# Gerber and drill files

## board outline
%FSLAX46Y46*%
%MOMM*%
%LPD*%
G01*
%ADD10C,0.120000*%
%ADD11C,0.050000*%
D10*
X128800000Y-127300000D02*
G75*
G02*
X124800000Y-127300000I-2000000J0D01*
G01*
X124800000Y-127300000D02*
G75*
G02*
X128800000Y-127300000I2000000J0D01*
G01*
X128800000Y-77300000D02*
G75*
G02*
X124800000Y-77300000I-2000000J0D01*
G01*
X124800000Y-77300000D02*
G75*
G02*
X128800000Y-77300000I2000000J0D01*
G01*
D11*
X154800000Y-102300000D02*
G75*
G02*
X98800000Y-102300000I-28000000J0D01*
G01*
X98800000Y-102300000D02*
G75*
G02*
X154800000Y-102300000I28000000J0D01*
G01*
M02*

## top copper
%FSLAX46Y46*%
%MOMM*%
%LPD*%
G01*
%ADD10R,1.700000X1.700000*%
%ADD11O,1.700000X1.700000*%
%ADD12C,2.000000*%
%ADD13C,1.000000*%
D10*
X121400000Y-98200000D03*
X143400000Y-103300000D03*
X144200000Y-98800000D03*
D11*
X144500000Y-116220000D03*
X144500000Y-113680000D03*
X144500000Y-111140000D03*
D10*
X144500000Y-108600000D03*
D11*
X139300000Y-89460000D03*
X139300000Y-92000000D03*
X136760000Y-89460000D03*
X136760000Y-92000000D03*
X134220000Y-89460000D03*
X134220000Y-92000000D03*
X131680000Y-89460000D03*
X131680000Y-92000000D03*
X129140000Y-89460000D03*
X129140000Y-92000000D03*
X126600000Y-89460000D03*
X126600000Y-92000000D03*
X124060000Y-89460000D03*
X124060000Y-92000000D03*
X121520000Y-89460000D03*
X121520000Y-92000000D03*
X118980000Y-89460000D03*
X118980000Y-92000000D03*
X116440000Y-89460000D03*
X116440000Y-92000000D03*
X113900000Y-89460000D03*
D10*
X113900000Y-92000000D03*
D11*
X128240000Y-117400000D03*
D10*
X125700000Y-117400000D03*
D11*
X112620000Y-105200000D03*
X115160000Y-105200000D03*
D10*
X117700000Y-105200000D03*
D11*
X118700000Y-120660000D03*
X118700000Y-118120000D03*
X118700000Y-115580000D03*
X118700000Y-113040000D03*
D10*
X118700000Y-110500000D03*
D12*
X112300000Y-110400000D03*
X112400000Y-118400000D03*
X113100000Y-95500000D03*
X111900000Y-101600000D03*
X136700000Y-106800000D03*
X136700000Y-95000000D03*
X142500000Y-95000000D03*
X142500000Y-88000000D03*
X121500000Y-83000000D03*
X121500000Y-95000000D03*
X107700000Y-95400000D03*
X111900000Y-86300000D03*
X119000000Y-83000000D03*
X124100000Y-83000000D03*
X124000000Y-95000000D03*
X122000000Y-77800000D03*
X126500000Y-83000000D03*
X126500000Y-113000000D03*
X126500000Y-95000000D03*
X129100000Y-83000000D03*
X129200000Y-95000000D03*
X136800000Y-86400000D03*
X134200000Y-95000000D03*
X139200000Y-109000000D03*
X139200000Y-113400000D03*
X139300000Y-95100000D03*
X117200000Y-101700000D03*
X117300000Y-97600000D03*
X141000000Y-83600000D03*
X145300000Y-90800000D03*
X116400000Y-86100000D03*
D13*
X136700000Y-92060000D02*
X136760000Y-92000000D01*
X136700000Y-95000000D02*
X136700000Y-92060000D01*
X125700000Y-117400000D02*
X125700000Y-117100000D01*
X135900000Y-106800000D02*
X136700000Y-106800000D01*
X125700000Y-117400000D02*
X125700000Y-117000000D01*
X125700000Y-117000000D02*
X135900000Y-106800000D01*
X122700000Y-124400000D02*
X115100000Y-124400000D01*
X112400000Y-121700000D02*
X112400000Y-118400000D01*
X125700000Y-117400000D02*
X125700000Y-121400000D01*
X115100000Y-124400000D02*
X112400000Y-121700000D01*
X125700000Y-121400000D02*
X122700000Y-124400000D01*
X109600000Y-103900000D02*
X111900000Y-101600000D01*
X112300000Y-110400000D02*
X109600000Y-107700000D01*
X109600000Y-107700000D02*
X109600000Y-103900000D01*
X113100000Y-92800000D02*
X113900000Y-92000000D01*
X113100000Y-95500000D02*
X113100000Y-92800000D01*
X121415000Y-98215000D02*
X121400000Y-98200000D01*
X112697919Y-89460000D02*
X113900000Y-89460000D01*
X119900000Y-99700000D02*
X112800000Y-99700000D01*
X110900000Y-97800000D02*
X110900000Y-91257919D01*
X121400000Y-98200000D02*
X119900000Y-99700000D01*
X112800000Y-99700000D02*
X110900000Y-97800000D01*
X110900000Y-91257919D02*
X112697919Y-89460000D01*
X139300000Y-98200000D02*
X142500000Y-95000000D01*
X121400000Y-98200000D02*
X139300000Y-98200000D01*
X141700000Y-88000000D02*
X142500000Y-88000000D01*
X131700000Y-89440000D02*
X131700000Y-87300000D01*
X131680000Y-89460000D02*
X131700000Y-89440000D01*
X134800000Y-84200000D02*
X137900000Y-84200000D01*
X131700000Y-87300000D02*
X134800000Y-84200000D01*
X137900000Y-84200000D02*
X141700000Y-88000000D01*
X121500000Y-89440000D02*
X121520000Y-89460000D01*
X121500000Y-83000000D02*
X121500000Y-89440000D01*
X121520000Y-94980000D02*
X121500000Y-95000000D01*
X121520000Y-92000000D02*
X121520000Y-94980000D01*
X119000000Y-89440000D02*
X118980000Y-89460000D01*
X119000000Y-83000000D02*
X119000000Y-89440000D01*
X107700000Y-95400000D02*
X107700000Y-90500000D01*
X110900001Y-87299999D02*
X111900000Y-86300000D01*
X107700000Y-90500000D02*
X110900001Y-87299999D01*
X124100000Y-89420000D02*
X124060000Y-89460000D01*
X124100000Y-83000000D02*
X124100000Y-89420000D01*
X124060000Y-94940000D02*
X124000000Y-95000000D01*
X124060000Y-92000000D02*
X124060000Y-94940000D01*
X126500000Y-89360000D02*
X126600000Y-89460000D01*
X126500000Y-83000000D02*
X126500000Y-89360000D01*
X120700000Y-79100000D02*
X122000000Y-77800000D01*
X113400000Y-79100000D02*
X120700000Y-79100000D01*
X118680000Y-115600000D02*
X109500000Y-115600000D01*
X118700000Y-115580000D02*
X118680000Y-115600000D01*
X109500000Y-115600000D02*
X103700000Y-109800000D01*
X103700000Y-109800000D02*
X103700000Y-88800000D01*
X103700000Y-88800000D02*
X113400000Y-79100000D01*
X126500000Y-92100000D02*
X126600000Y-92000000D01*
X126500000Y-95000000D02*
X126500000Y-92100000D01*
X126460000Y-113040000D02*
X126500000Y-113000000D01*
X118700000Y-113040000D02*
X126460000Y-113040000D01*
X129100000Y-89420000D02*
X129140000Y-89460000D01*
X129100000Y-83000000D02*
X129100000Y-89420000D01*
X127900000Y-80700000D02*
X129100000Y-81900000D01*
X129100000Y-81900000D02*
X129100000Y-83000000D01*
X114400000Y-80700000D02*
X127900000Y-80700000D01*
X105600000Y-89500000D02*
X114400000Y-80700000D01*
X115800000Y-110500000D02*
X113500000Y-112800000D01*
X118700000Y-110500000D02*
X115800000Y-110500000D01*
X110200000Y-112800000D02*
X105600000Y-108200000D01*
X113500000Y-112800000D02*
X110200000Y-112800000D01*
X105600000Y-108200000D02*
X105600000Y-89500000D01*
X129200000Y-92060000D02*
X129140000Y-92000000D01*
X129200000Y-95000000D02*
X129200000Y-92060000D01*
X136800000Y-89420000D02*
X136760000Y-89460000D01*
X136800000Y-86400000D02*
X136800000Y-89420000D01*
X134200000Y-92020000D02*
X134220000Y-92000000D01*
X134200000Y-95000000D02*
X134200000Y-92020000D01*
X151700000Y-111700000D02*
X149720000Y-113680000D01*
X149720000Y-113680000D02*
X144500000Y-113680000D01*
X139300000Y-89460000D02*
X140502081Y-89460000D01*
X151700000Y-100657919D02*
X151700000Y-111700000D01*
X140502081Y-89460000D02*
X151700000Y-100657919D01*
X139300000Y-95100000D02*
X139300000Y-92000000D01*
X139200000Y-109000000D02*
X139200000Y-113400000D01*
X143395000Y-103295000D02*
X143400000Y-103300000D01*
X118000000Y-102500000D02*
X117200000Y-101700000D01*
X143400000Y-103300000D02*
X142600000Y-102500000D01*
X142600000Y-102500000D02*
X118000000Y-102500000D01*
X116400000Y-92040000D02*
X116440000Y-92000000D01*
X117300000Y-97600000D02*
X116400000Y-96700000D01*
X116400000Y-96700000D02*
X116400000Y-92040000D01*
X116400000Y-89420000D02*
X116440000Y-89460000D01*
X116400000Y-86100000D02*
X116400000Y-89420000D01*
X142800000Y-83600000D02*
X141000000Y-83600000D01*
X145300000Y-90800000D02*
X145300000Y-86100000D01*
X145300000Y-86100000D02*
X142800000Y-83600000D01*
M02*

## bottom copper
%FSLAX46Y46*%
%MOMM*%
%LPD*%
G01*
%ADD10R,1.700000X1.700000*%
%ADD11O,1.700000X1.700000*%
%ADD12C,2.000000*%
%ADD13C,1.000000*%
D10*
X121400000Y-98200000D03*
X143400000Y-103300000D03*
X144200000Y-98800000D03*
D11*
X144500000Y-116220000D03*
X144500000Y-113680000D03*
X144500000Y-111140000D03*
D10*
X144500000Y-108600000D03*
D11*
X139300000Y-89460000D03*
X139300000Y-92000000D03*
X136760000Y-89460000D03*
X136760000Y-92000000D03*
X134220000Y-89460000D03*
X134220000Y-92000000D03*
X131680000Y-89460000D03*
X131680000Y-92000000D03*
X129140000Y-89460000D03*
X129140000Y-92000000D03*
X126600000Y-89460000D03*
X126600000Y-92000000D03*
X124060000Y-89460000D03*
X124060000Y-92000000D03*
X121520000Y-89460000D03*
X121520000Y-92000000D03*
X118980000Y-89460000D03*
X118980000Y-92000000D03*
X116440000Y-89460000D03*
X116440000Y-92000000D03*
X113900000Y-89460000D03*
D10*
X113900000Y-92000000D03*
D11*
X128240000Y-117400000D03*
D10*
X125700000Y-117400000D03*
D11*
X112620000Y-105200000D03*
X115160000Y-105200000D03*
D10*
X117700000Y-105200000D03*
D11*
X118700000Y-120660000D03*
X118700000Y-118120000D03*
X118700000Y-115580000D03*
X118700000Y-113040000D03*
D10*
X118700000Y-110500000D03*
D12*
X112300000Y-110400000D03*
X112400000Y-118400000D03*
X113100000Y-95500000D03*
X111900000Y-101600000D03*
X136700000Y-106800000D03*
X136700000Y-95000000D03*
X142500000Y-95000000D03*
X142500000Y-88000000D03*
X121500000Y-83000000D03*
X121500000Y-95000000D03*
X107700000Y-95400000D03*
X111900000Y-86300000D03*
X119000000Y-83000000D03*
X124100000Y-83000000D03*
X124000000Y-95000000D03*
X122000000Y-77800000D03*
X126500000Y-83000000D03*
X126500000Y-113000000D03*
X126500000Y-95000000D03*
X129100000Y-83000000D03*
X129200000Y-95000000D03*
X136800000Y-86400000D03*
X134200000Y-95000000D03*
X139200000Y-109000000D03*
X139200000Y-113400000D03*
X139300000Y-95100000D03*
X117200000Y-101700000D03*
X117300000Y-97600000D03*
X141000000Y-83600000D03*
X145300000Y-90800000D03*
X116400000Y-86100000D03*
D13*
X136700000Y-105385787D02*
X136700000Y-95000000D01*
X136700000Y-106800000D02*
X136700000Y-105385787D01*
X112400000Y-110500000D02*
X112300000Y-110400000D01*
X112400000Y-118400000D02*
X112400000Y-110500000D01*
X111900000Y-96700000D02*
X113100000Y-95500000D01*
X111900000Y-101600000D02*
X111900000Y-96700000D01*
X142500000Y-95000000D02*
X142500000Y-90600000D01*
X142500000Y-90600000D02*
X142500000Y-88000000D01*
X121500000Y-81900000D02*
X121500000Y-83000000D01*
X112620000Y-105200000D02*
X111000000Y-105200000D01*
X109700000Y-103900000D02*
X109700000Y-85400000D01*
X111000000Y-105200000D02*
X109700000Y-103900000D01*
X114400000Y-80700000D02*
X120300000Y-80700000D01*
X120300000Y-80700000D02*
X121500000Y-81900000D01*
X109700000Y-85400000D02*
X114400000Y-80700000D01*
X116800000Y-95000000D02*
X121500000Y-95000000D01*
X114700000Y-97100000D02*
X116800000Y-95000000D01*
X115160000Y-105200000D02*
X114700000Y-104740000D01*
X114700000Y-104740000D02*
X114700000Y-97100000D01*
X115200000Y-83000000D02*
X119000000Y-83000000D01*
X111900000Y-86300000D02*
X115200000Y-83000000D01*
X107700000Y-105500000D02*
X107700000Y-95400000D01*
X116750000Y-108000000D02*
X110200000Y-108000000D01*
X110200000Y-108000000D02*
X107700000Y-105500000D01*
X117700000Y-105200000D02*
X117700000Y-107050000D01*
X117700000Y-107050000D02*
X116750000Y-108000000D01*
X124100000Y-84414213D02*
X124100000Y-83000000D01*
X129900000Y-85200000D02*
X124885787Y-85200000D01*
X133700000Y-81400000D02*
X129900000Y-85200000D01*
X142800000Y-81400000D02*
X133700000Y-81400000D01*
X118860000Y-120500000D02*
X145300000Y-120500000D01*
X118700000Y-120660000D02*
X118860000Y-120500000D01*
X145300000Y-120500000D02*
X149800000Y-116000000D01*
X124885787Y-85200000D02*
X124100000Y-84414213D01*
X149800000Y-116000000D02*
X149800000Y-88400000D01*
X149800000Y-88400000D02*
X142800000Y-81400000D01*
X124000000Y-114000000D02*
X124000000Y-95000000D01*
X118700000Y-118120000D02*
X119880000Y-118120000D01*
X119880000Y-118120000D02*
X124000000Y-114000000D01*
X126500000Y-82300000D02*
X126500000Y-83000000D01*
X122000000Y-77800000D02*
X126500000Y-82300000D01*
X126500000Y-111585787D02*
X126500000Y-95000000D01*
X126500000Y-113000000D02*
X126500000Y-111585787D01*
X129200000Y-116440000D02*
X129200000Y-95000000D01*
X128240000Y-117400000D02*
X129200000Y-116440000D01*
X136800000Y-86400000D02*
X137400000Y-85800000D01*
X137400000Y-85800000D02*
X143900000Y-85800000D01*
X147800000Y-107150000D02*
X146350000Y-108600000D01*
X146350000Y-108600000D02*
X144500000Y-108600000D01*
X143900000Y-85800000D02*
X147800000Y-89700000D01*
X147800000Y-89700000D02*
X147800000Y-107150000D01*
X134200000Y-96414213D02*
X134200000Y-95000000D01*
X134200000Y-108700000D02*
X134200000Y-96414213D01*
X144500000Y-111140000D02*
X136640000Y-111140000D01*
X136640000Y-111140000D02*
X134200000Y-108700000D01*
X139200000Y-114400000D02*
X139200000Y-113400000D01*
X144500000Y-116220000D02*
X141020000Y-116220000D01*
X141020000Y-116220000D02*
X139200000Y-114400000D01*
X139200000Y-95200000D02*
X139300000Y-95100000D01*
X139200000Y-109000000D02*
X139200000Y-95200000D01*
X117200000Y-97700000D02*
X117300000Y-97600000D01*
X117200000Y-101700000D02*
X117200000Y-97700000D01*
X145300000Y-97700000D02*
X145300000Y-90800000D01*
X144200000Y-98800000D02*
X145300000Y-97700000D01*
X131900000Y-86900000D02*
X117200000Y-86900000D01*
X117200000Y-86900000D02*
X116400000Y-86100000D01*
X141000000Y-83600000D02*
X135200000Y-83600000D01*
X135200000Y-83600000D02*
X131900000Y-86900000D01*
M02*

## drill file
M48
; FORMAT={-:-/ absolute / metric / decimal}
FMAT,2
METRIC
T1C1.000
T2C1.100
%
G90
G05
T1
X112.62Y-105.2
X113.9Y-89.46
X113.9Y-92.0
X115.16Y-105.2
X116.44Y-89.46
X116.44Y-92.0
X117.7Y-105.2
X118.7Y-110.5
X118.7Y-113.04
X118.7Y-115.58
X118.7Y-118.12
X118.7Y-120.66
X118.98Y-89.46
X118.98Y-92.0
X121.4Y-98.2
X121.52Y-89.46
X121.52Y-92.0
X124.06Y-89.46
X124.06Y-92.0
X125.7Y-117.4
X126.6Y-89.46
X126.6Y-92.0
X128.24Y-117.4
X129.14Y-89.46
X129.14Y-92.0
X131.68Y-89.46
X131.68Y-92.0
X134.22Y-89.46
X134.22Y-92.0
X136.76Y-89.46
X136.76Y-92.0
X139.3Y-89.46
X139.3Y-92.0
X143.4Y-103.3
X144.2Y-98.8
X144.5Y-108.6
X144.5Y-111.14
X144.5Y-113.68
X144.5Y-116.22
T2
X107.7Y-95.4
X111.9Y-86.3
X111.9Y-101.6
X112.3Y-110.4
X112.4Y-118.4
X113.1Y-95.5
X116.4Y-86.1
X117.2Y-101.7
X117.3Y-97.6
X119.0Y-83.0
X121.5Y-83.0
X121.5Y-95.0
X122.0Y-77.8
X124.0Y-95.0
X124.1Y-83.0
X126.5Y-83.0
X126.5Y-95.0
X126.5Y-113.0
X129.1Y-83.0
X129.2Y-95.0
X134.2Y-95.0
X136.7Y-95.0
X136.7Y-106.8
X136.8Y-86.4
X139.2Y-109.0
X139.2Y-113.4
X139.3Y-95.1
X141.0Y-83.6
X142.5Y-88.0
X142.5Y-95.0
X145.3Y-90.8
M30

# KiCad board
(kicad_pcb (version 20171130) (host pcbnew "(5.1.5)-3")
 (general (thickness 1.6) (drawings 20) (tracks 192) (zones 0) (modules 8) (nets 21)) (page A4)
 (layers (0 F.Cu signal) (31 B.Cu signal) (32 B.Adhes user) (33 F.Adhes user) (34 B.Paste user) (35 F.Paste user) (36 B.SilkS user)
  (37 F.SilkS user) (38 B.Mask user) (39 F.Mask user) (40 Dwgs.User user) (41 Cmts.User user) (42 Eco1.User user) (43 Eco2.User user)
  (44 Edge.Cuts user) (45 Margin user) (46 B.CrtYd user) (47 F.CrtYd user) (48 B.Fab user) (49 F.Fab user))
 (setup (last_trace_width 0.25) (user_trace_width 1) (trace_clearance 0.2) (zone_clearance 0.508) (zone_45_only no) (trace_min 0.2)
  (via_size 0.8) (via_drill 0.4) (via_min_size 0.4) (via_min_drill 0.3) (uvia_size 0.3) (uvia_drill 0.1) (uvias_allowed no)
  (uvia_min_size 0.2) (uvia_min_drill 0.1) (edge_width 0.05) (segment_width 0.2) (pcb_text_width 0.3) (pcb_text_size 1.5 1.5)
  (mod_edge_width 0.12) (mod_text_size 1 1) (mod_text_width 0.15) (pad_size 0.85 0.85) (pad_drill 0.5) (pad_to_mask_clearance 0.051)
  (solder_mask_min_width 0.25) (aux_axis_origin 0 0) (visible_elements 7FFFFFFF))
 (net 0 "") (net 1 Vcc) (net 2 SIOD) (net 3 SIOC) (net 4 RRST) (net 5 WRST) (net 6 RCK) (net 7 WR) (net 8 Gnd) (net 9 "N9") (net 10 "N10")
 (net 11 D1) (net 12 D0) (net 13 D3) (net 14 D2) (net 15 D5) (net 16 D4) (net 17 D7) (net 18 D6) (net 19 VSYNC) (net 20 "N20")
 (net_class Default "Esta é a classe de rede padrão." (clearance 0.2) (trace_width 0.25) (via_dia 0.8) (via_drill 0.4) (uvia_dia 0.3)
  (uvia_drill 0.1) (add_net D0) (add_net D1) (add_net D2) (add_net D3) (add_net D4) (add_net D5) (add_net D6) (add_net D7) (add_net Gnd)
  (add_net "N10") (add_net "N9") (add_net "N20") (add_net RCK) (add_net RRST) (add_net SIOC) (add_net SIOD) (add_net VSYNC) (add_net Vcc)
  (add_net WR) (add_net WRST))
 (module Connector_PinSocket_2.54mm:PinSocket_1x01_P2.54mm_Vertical (layer F.Cu) (at 121.4 98.2)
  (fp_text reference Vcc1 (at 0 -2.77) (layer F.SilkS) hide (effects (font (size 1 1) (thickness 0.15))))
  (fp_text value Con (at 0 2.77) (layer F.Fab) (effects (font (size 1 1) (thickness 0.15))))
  (pad 1 thru_hole rect (at 0 0) (size 1.7 1.7) (drill 1) (layers *.Cu *.Mask) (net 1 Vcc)))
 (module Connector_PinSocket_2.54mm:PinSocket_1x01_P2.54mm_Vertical (layer F.Cu) (at 143.4 103.3)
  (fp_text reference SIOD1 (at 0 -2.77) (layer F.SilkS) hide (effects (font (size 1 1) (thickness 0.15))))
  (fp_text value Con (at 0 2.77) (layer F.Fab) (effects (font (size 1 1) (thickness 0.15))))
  (pad 1 thru_hole rect (at 0 0) (size 1.7 1.7) (drill 1) (layers *.Cu *.Mask) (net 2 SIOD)))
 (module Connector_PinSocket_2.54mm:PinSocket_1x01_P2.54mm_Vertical (layer F.Cu) (at 144.2 98.8)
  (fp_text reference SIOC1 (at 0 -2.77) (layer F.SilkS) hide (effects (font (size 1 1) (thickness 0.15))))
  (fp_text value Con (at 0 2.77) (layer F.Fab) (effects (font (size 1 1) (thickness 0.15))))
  (pad 1 thru_hole rect (at 0 0) (size 1.7 1.7) (drill 1) (layers *.Cu *.Mask) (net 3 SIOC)))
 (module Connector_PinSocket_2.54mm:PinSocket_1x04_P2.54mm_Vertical (layer F.Cu) (at 144.5 108.6)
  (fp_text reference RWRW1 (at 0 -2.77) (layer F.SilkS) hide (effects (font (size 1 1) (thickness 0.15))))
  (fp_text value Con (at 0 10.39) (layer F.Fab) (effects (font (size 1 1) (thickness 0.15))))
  (pad 4 thru_hole oval (at 0 7.62) (size 1.7 1.7) (drill 1) (layers *.Cu *.Mask) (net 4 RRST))
  (pad 3 thru_hole oval (at 0 5.08) (size 1.7 1.7) (drill 1) (layers *.Cu *.Mask) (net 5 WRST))
  (pad 2 thru_hole oval (at 0 2.54) (size 1.7 1.7) (drill 1) (layers *.Cu *.Mask) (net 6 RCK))
  (pad 1 thru_hole rect (at 0 0) (size 1.7 1.7) (drill 1) (layers *.Cu *.Mask) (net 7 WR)))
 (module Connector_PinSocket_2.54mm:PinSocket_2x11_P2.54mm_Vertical (layer B.Cu) (at 113.9 92 270)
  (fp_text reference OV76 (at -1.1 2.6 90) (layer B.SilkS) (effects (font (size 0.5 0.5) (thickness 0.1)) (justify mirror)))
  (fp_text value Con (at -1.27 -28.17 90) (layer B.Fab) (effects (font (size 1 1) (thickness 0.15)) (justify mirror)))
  (pad 22 thru_hole oval (at -2.54 -25.4 270) (size 1.7 1.7) (drill 1) (layers *.Cu *.Mask) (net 5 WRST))
  (pad 21 thru_hole oval (at 0 -25.4 270) (size 1.7 1.7) (drill 1) (layers *.Cu *.Mask) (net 4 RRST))
  (pad 20 thru_hole oval (at -2.54 -22.86 270) (size 1.7 1.7) (drill 1) (layers *.Cu *.Mask) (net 7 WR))
  (pad 19 thru_hole oval (at 0 -22.86 270) (size 1.7 1.7) (drill 1) (layers *.Cu *.Mask) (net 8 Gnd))
  (pad 18 thru_hole oval (at -2.54 -20.32 270) (size 1.7 1.7) (drill 1) (layers *.Cu *.Mask) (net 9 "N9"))
  (pad 17 thru_hole oval (at 0 -20.32 270) (size 1.7 1.7) (drill 1) (layers *.Cu *.Mask) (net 6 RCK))
  (pad 16 thru_hole oval (at -2.54 -17.78 270) (size 1.7 1.7) (drill 1) (layers *.Cu *.Mask) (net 1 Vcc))
  (pad 15 thru_hole oval (at 0 -17.78 270) (size 1.7 1.7) (drill 1) (layers *.Cu *.Mask) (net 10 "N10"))
  (pad 14 thru_hole oval (at -2.54 -15.24 270) (size 1.7 1.7) (drill 1) (layers *.Cu *.Mask) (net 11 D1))
  (pad 13 thru_hole oval (at 0 -15.24 270) (size 1.7 1.7) (drill 1) (layers *.Cu *.Mask) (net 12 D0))
  (pad 12 thru_hole oval (at -2.54 -12.7 270) (size 1.7 1.7) (drill 1) (layers *.Cu *.Mask) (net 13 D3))
  (pad 11 thru_hole oval (at 0 -12.7 270) (size 1.7 1.7) (drill 1) (layers *.Cu *.Mask) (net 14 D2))
  (pad 10 thru_hole oval (at -2.54 -10.16 270) (size 1.7 1.7) (drill 1) (layers *.Cu *.Mask) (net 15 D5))
  (pad 9 thru_hole oval (at 0 -10.16 270) (size 1.7 1.7) (drill 1) (layers *.Cu *.Mask) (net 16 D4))
  (pad 8 thru_hole oval (at -2.54 -7.62 270) (size 1.7 1.7) (drill 1) (layers *.Cu *.Mask) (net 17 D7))
  (pad 7 thru_hole oval (at 0 -7.62 270) (size 1.7 1.7) (drill 1) (layers *.Cu *.Mask) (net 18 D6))
  (pad 6 thru_hole oval (at -2.54 -5.08 270) (size 1.7 1.7) (drill 1) (layers *.Cu *.Mask) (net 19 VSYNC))
  (pad 5 thru_hole oval (at 0 -5.08 270) (size 1.7 1.7) (drill 1) (layers *.Cu *.Mask) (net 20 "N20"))
  (pad 4 thru_hole oval (at -2.54 -2.54 270) (size 1.7 1.7) (drill 1) (layers *.Cu *.Mask) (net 3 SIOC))
  (pad 3 thru_hole oval (at 0 -2.54 270) (size 1.7 1.7) (drill 1) (layers *.Cu *.Mask) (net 2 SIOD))
  (pad 2 thru_hole oval (at -2.54 0 270) (size 1.7 1.7) (drill 1) (layers *.Cu *.Mask) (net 1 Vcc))
  (pad 1 thru_hole rect (at 0 0 270) (size 1.7 1.7) (drill 1) (layers *.Cu *.Mask) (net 8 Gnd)))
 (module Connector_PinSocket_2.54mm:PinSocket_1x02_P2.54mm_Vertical (layer F.Cu) (at 125.7 117.4 90)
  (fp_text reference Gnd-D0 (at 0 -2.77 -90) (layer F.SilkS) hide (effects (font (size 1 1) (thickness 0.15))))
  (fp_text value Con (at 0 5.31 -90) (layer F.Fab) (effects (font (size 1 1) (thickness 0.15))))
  (pad 2 thru_hole oval (at 0 2.54 90) (size 1.7 1.7) (drill 1) (layers *.Cu *.Mask) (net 12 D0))
  (pad 1 thru_hole rect (at 0 0 90) (size 1.7 1.7) (drill 1) (layers *.Cu *.Mask) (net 8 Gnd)))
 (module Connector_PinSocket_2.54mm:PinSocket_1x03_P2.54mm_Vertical (layer F.Cu) (at 117.7 105.2 270)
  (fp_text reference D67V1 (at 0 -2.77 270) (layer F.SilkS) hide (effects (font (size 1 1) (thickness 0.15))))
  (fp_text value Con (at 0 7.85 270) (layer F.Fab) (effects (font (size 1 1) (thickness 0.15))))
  (pad 3 thru_hole oval (at 0 5.08 270) (size 1.7 1.7) (drill 1) (layers *.Cu *.Mask) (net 17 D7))
  (pad 2 thru_hole oval (at 0 2.54 270) (size 1.7 1.7) (drill 1) (layers *.Cu *.Mask) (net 18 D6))
  (pad 1 thru_hole rect (at 0 0 270) (size 1.7 1.7) (drill 1) (layers *.Cu *.Mask) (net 19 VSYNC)))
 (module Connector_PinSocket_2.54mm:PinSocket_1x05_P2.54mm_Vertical (layer F.Cu) (at 118.7 110.5)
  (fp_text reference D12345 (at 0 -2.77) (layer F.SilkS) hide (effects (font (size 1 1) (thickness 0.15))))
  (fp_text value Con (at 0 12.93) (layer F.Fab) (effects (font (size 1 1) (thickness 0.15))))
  (pad 5 thru_hole oval (at 0 10.16) (size 1.7 1.7) (drill 1) (layers *.Cu *.Mask) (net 15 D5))
  (pad 4 thru_hole oval (at 0 7.62) (size 1.7 1.7) (drill 1) (layers *.Cu *.Mask) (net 16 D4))
  (pad 3 thru_hole oval (at 0 5.08) (size 1.7 1.7) (drill 1) (layers *.Cu *.Mask) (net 13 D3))
  (pad 2 thru_hole oval (at 0 2.54) (size 1.7 1.7) (drill 1) (layers *.Cu *.Mask) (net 14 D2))
  (pad 1 thru_hole rect (at 0 0) (size 1.7 1.7) (drill 1) (layers *.Cu *.Mask) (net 11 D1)))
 (gr_circle (center 126.8 127.3) (end 128.8 127.3) (layer Edge.Cuts) (width 0.12))
 (gr_circle (center 126.8 77.3) (end 128.8 77.3) (layer Edge.Cuts) (width 0.12))
 (gr_circle (center 126.8 102.3) (end 154.8 102.3) (layer Edge.Cuts) (width 0.05))
 (via (at 112.3 110.4) (size 2) (drill 1.1) (layers F.Cu B.Cu) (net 8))
 (via (at 112.4 118.4) (size 2) (drill 1.1) (layers F.Cu B.Cu) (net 8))
 (via (at 113.1 95.5) (size 2) (drill 1.1) (layers F.Cu B.Cu) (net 8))
 (via (at 111.9 101.6) (size 2) (drill 1.1) (layers F.Cu B.Cu) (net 8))
 (via (at 136.7 106.8) (size 2) (drill 1.1) (layers F.Cu B.Cu) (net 8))
 (via (at 136.7 95) (size 2) (drill 1.1) (layers F.Cu B.Cu) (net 8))
 (segment (start 136.7 92.06) (end 136.76 92) (width 1) (layer F.Cu) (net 8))
 (segment (start 136.7 95) (end 136.7 92.06) (width 1) (layer F.Cu) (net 8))
 (segment (start 125.7 117.4) (end 125.7 117.1) (width 1) (layer F.Cu) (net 8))
 (segment (start 135.9 106.8) (end 136.7 106.8) (width 1) (layer F.Cu) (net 8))
 (segment (start 125.7 117.4) (end 125.7 117) (width 1) (layer F.Cu) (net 8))
 (segment (start 125.7 117) (end 135.9 106.8) (width 1) (layer F.Cu) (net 8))
 (segment (start 136.7 105.385787) (end 136.7 95) (width 1) (layer B.Cu) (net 8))
 (segment (start 136.7 106.8) (end 136.7 105.385787) (width 1) (layer B.Cu) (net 8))
 (segment (start 122.7 124.4) (end 115.1 124.4) (width 1) (layer F.Cu) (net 8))
 (segment (start 112.4 121.7) (end 112.4 118.4) (width 1) (layer F.Cu) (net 8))
 (segment (start 125.7 117.4) (end 125.7 121.4) (width 1) (layer F.Cu) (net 8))
 (segment (start 115.1 124.4) (end 112.4 121.7) (width 1) (layer F.Cu) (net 8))
 (segment (start 125.7 121.4) (end 122.7 124.4) (width 1) (layer F.Cu) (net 8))
 (segment (start 112.4 110.5) (end 112.3 110.4) (width 1) (layer B.Cu) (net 8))
 (segment (start 112.4 118.4) (end 112.4 110.5) (width 1) (layer B.Cu) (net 8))
 (segment (start 109.6 103.9) (end 111.9 101.6) (width 1) (layer F.Cu) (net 8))
 (segment (start 112.3 110.4) (end 109.6 107.7) (width 1) (layer F.Cu) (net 8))
 (segment (start 109.6 107.7) (end 109.6 103.9) (width 1) (layer F.Cu) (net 8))
 (segment (start 111.9 96.7) (end 113.1 95.5) (width 1) (layer B.Cu) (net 8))
 (segment (start 111.9 101.6) (end 111.9 96.7) (width 1) (layer B.Cu) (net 8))
 (segment (start 113.1 92.8) (end 113.9 92) (width 1) (layer F.Cu) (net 8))
 (segment (start 113.1 95.5) (end 113.1 92.8) (width 1) (layer F.Cu) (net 8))
 (via (at 142.5 95) (size 2) (drill 1.1) (layers F.Cu B.Cu) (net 1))
 (via (at 142.5 88) (size 2) (drill 1.1) (layers F.Cu B.Cu) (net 1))
 (segment (start 121.415 98.215) (end 121.4 98.2) (width 1) (layer F.Cu) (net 1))
 (segment (start 112.697919 89.46) (end 113.9 89.46) (width 1) (layer F.Cu) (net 1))
 (segment (start 119.9 99.7) (end 112.8 99.7) (width 1) (layer F.Cu) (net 1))
 (segment (start 110.9 97.8) (end 110.9 91.257919) (width 1) (layer F.Cu) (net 1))
 (segment (start 121.4 98.2) (end 119.9 99.7) (width 1) (layer F.Cu) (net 1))
 (segment (start 112.8 99.7) (end 110.9 97.8) (width 1) (layer F.Cu) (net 1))
 (segment (start 110.9 91.257919) (end 112.697919 89.46) (width 1) (layer F.Cu) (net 1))
 (segment (start 139.3 98.2) (end 142.5 95) (width 1) (layer F.Cu) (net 1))
 (segment (start 121.4 98.2) (end 139.3 98.2) (width 1) (layer F.Cu) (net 1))
 (segment (start 142.5 95) (end 142.5 90.6) (width 1) (layer B.Cu) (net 1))
 (segment (start 142.5 90.6) (end 142.5 88) (width 1) (layer B.Cu) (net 1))
 (segment (start 141.7 88) (end 142.5 88) (width 1) (layer F.Cu) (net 1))
 (segment (start 131.7 89.44) (end 131.7 87.3) (width 1) (layer F.Cu) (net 1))
 (segment (start 131.68 89.46) (end 131.7 89.44) (width 1) (layer F.Cu) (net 1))
 (segment (start 134.8 84.2) (end 137.9 84.2) (width 1) (layer F.Cu) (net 1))
 (segment (start 131.7 87.3) (end 134.8 84.2) (width 1) (layer F.Cu) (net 1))
 (segment (start 137.9 84.2) (end 141.7 88) (width 1) (layer F.Cu) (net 1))
 (via (at 121.5 83) (size 2) (drill 1.1) (layers F.Cu B.Cu) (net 17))
 (segment (start 121.5 89.44) (end 121.52 89.46) (width 1) (layer F.Cu) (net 17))
 (segment (start 121.5 83) (end 121.5 89.44) (width 1) (layer F.Cu) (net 17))
 (segment (start 121.5 81.9) (end 121.5 83) (width 1) (layer B.Cu) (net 17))
 (segment (start 112.62 105.2) (end 111 105.2) (width 1) (layer B.Cu) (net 17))
 (segment (start 109.7 103.9) (end 109.7 85.4) (width 1) (layer B.Cu) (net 17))
 (segment (start 111 105.2) (end 109.7 103.9) (width 1) (layer B.Cu) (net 17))
 (segment (start 114.4 80.7) (end 120.3 80.7) (width 1) (layer B.Cu) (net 17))
 (segment (start 120.3 80.7) (end 121.5 81.9) (width 1) (layer B.Cu) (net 17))
 (segment (start 109.7 85.4) (end 114.4 80.7) (width 1) (layer B.Cu) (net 17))
 (via (at 121.5 95) (size 2) (drill 1.1) (layers F.Cu B.Cu) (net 18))
 (segment (start 121.52 94.98) (end 121.5 95) (width 1) (layer F.Cu) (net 18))
 (segment (start 121.52 92) (end 121.52 94.98) (width 1) (layer F.Cu) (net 18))
 (segment (start 116.8 95) (end 121.5 95) (width 1) (layer B.Cu) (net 18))
 (segment (start 114.7 97.1) (end 116.8 95) (width 1) (layer B.Cu) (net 18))
 (segment (start 115.16 105.2) (end 114.7 104.74) (width 1) (layer B.Cu) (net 18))
 (segment (start 114.7 104.74) (end 114.7 97.1) (width 1) (layer B.Cu) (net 18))
 (via (at 107.7 95.4) (size 2) (drill 1.1) (layers F.Cu B.Cu) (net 19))
 (via (at 111.9 86.3) (size 2) (drill 1.1) (layers F.Cu B.Cu) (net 19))
 (via (at 119 83) (size 2) (drill 1.1) (layers F.Cu B.Cu) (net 19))
 (segment (start 119 89.44) (end 118.98 89.46) (width 1) (layer F.Cu) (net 19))
 (segment (start 119 83) (end 119 89.44) (width 1) (layer F.Cu) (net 19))
 (segment (start 107.7 95.4) (end 107.7 90.5) (width 1) (layer F.Cu) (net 19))
 (segment (start 110.900001 87.299999) (end 111.9 86.3) (width 1) (layer F.Cu) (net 19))
 (segment (start 107.7 90.5) (end 110.900001 87.299999) (width 1) (layer F.Cu) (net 19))
 (segment (start 115.2 83) (end 119 83) (width 1) (layer B.Cu) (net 19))
 (segment (start 111.9 86.3) (end 115.2 83) (width 1) (layer B.Cu) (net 19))
 (segment (start 107.7 105.5) (end 107.7 95.4) (width 1) (layer B.Cu) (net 19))
 (segment (start 116.75 108) (end 110.2 108) (width 1) (layer B.Cu) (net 19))
 (segment (start 110.2 108) (end 107.7 105.5) (width 1) (layer B.Cu) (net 19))
 (segment (start 117.7 105.2) (end 117.7 107.05) (width 1) (layer B.Cu) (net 19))
 (segment (start 117.7 107.05) (end 116.75 108) (width 1) (layer B.Cu) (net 19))
 (via (at 124.1 83) (size 2) (drill 1.1) (layers F.Cu B.Cu) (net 15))
 (segment (start 124.1 89.42) (end 124.06 89.46) (width 1) (layer F.Cu) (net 15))
 (segment (start 124.1 83) (end 124.1 89.42) (width 1) (layer F.Cu) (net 15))
 (segment (start 124.1 84.414213) (end 124.1 83) (width 1) (layer B.Cu) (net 15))
 (segment (start 129.9 85.2) (end 124.885787 85.2) (width 1) (layer B.Cu) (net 15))
 (segment (start 133.7 81.4) (end 129.9 85.2) (width 1) (layer B.Cu) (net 15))
 (segment (start 142.8 81.4) (end 133.7 81.4) (width 1) (layer B.Cu) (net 15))
 (segment (start 118.86 120.5) (end 145.3 120.5) (width 1) (layer B.Cu) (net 15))
 (segment (start 118.7 120.66) (end 118.86 120.5) (width 1) (layer B.Cu) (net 15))
 (segment (start 145.3 120.5) (end 149.8 116) (width 1) (layer B.Cu) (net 15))
 (segment (start 124.885787 85.2) (end 124.1 84.414213) (width 1) (layer B.Cu) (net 15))
 (segment (start 149.8 116) (end 149.8 88.4) (width 1) (layer B.Cu) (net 15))
 (segment (start 149.8 88.4) (end 142.8 81.4) (width 1) (layer B.Cu) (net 15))
 (via (at 124 95) (size 2) (drill 1.1) (layers F.Cu B.Cu) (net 16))
 (segment (start 124 114) (end 124 95) (width 1) (layer B.Cu) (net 16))
 (segment (start 118.7 118.12) (end 119.88 118.12) (width 1) (layer B.Cu) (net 16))
 (segment (start 119.88 118.12) (end 124 114) (width 1) (layer B.Cu) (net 16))
 (segment (start 124.06 94.94) (end 124 95) (width 1) (layer F.Cu) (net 16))
 (segment (start 124.06 92) (end 124.06 94.94) (width 1) (layer F.Cu) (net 16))
 (via (at 122 77.8) (size 2) (drill 1.1) (layers F.Cu B.Cu) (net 13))
 (via (at 126.5 83) (size 2) (drill 1.1) (layers F.Cu B.Cu) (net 13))
 (segment (start 126.5 89.36) (end 126.6 89.46) (width 1) (layer F.Cu) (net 13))
 (segment (start 126.5 83) (end 126.5 89.36) (width 1) (layer F.Cu) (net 13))
 (segment (start 126.5 82.3) (end 126.5 83) (width 1) (layer B.Cu) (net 13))
 (segment (start 122 77.8) (end 126.5 82.3) (width 1) (layer B.Cu) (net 13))
 (segment (start 120.7 79.1) (end 122 77.8) (width 1) (layer F.Cu) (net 13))
 (segment (start 113.4 79.1) (end 120.7 79.1) (width 1) (layer F.Cu) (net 13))
 (segment (start 118.68 115.6) (end 109.5 115.6) (width 1) (layer F.Cu) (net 13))
 (segment (start 118.7 115.58) (end 118.68 115.6) (width 1) (layer F.Cu) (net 13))
 (segment (start 109.5 115.6) (end 103.7 109.8) (width 1) (layer F.Cu) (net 13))
 (segment (start 103.7 109.8) (end 103.7 88.8) (width 1) (layer F.Cu) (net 13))
 (segment (start 103.7 88.8) (end 113.4 79.1) (width 1) (layer F.Cu) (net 13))
 (via (at 126.5 113) (size 2) (drill 1.1) (layers F.Cu B.Cu) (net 14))
 (via (at 126.5 95) (size 2) (drill 1.1) (layers F.Cu B.Cu) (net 14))
 (segment (start 126.5 92.1) (end 126.6 92) (width 1) (layer F.Cu) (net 14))
 (segment (start 126.5 95) (end 126.5 92.1) (width 1) (layer F.Cu) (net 14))
 (segment (start 126.46 113.04) (end 126.5 113) (width 1) (layer F.Cu) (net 14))
 (segment (start 118.7 113.04) (end 126.46 113.04) (width 1) (layer F.Cu) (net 14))
 (segment (start 126.5 111.585787) (end 126.5 95) (width 1) (layer B.Cu) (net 14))
 (segment (start 126.5 113) (end 126.5 111.585787) (width 1) (layer B.Cu) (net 14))
 (via (at 129.1 83) (size 2) (drill 1.1) (layers F.Cu B.Cu) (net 11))
 (segment (start 129.1 89.42) (end 129.14 89.46) (width 1) (layer F.Cu) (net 11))
 (segment (start 129.1 83) (end 129.1 89.42) (width 1) (layer F.Cu) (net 11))
 (segment (start 127.9 80.7) (end 129.1 81.9) (width 1) (layer F.Cu) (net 11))
 (segment (start 129.1 81.9) (end 129.1 83) (width 1) (layer F.Cu) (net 11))
 (segment (start 114.4 80.7) (end 127.9 80.7) (width 1) (layer F.Cu) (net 11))
 (segment (start 105.6 89.5) (end 114.4 80.7) (width 1) (layer F.Cu) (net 11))
 (segment (start 115.8 110.5) (end 113.5 112.8) (width 1) (layer F.Cu) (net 11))
 (segment (start 118.7 110.5) (end 115.8 110.5) (width 1) (layer F.Cu) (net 11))
 (segment (start 110.2 112.8) (end 105.6 108.2) (width 1) (layer F.Cu) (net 11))
 (segment (start 113.5 112.8) (end 110.2 112.8) (width 1) (layer F.Cu) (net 11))
 (segment (start 105.6 108.2) (end 105.6 89.5) (width 1) (layer F.Cu) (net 11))
 (via (at 129.2 95) (size 2) (drill 1.1) (layers F.Cu B.Cu) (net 12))
 (segment (start 129.2 92.06) (end 129.14 92) (width 1) (layer F.Cu) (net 12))
 (segment (start 129.2 95) (end 129.2 92.06) (width 1) (layer F.Cu) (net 12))
 (segment (start 129.2 116.44) (end 129.2 95) (width 1) (layer B.Cu) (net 12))
 (segment (start 128.24 117.4) (end 129.2 116.44) (width 1) (layer B.Cu) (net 12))
 (via (at 136.8 86.4) (size 2) (drill 1.1) (layers F.Cu B.Cu) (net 7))
 (segment (start 136.8 89.42) (end 136.76 89.46) (width 1) (layer F.Cu) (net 7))
 (segment (start 136.8 86.4) (end 136.8 89.42) (width 1) (layer F.Cu) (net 7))
 (segment (start 136.8 86.4) (end 137.4 85.8) (width 1) (layer B.Cu) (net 7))
 (segment (start 137.4 85.8) (end 143.9 85.8) (width 1) (layer B.Cu) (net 7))
 (segment (start 147.8 107.15) (end 146.35 108.6) (width 1) (layer B.Cu) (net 7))
 (segment (start 146.35 108.6) (end 144.5 108.6) (width 1) (layer B.Cu) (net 7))
 (segment (start 143.9 85.8) (end 147.8 89.7) (width 1) (layer B.Cu) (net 7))
 (segment (start 147.8 89.7) (end 147.8 107.15) (width 1) (layer B.Cu) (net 7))
 (via (at 134.2 95) (size 2) (drill 1.1) (layers F.Cu B.Cu) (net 6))
 (segment (start 134.2 96.414213) (end 134.2 95) (width 1) (layer B.Cu) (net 6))
 (segment (start 134.2 108.7) (end 134.2 96.414213) (width 1) (layer B.Cu) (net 6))
 (segment (start 144.5 111.14) (end 136.64 111.14) (width 1) (layer B.Cu) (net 6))
 (segment (start 136.64 111.14) (end 134.2 108.7) (width 1) (layer B.Cu) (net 6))
 (segment (start 134.2 92.02) (end 134.22 92) (width 1) (layer F.Cu) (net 6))
 (segment (start 134.2 95) (end 134.2 92.02) (width 1) (layer F.Cu) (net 6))
 (segment (start 151.7 111.7) (end 149.72 113.68) (width 1) (layer F.Cu) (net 5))
 (segment (start 149.72 113.68) (end 144.5 113.68) (width 1) (layer F.Cu) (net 5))
 (segment (start 139.3 89.46) (end 140.502081 89.46) (width 1) (layer F.Cu) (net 5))
 (segment (start 151.7 100.657919) (end 151.7 111.7) (width 1) (layer F.Cu) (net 5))
 (segment (start 140.502081 89.46) (end 151.7 100.657919) (width 1) (layer F.Cu) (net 5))
 (via (at 139.2 109) (size 2) (drill 1.1) (layers F.Cu B.Cu) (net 4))
 (via (at 139.2 113.4) (size 2) (drill 1.1) (layers F.Cu B.Cu) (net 4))
 (via (at 139.3 95.1) (size 2) (drill 1.1) (layers F.Cu B.Cu) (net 4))
 (segment (start 139.2 114.4) (end 139.2 113.4) (width 1) (layer B.Cu) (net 4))
 (segment (start 144.5 116.22) (end 141.02 116.22) (width 1) (layer B.Cu) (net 4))
 (segment (start 141.02 116.22) (end 139.2 114.4) (width 1) (layer B.Cu) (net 4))
 (segment (start 139.2 95.2) (end 139.3 95.1) (width 1) (layer B.Cu) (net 4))
 (segment (start 139.2 109) (end 139.2 95.2) (width 1) (layer B.Cu) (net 4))
 (segment (start 139.3 95.1) (end 139.3 92) (width 1) (layer F.Cu) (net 4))
 (segment (start 139.2 109) (end 139.2 113.4) (width 1) (layer F.Cu) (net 4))
 (via (at 117.2 101.7) (size 2) (drill 1.1) (layers F.Cu B.Cu) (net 2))
 (via (at 117.3 97.6) (size 2) (drill 1.1) (layers F.Cu B.Cu) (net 2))
 (segment (start 143.395 103.295) (end 143.4 103.3) (width 1) (layer F.Cu) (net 2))
 (segment (start 118 102.5) (end 117.2 101.7) (width 1) (layer F.Cu) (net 2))
 (segment (start 143.4 103.3) (end 142.6 102.5) (width 1) (layer F.Cu) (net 2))
 (segment (start 142.6 102.5) (end 118 102.5) (width 1) (layer F.Cu) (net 2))
 (segment (start 117.2 97.7) (end 117.3 97.6) (width 1) (layer B.Cu) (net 2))
 (segment (start 117.2 101.7) (end 117.2 97.7) (width 1) (layer B.Cu) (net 2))
 (segment (start 116.4 92.04) (end 116.44 92) (width 1) (layer F.Cu) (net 2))
 (segment (start 117.3 97.6) (end 116.4 96.7) (width 1) (layer F.Cu) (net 2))
 (segment (start 116.4 96.7) (end 116.4 92.04) (width 1) (layer F.Cu) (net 2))
 (via (at 141 83.6) (size 2) (drill 1.1) (layers F.Cu B.Cu) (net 3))
 (via (at 145.3 90.8) (size 2) (drill 1.1) (layers F.Cu B.Cu) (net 3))
 (via (at 116.4 86.1) (size 2) (drill 1.1) (layers F.Cu B.Cu) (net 3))
 (segment (start 116.4 89.42) (end 116.44 89.46) (width 1) (layer F.Cu) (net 3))
 (segment (start 116.4 86.1) (end 116.4 89.42) (width 1) (layer F.Cu) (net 3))
 (segment (start 145.3 97.7) (end 145.3 90.8) (width 1) (layer B.Cu) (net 3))
 (segment (start 144.2 98.8) (end 145.3 97.7) (width 1) (layer B.Cu) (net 3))
 (segment (start 142.8 83.6) (end 141 83.6) (width 1) (layer F.Cu) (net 3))
 (segment (start 145.3 90.8) (end 145.3 86.1) (width 1) (layer F.Cu) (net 3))
 (segment (start 145.3 86.1) (end 142.8 83.6) (width 1) (layer F.Cu) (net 3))
 (segment (start 131.9 86.9) (end 117.2 86.9) (width 1) (layer B.Cu) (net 3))
 (segment (start 117.2 86.9) (end 116.4 86.1) (width 1) (layer B.Cu) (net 3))
 (segment (start 141 83.6) (end 135.2 83.6) (width 1) (layer B.Cu) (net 3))
 (segment (start 135.2 83.6) (end 131.9 86.9) (width 1) (layer B.Cu) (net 3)))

